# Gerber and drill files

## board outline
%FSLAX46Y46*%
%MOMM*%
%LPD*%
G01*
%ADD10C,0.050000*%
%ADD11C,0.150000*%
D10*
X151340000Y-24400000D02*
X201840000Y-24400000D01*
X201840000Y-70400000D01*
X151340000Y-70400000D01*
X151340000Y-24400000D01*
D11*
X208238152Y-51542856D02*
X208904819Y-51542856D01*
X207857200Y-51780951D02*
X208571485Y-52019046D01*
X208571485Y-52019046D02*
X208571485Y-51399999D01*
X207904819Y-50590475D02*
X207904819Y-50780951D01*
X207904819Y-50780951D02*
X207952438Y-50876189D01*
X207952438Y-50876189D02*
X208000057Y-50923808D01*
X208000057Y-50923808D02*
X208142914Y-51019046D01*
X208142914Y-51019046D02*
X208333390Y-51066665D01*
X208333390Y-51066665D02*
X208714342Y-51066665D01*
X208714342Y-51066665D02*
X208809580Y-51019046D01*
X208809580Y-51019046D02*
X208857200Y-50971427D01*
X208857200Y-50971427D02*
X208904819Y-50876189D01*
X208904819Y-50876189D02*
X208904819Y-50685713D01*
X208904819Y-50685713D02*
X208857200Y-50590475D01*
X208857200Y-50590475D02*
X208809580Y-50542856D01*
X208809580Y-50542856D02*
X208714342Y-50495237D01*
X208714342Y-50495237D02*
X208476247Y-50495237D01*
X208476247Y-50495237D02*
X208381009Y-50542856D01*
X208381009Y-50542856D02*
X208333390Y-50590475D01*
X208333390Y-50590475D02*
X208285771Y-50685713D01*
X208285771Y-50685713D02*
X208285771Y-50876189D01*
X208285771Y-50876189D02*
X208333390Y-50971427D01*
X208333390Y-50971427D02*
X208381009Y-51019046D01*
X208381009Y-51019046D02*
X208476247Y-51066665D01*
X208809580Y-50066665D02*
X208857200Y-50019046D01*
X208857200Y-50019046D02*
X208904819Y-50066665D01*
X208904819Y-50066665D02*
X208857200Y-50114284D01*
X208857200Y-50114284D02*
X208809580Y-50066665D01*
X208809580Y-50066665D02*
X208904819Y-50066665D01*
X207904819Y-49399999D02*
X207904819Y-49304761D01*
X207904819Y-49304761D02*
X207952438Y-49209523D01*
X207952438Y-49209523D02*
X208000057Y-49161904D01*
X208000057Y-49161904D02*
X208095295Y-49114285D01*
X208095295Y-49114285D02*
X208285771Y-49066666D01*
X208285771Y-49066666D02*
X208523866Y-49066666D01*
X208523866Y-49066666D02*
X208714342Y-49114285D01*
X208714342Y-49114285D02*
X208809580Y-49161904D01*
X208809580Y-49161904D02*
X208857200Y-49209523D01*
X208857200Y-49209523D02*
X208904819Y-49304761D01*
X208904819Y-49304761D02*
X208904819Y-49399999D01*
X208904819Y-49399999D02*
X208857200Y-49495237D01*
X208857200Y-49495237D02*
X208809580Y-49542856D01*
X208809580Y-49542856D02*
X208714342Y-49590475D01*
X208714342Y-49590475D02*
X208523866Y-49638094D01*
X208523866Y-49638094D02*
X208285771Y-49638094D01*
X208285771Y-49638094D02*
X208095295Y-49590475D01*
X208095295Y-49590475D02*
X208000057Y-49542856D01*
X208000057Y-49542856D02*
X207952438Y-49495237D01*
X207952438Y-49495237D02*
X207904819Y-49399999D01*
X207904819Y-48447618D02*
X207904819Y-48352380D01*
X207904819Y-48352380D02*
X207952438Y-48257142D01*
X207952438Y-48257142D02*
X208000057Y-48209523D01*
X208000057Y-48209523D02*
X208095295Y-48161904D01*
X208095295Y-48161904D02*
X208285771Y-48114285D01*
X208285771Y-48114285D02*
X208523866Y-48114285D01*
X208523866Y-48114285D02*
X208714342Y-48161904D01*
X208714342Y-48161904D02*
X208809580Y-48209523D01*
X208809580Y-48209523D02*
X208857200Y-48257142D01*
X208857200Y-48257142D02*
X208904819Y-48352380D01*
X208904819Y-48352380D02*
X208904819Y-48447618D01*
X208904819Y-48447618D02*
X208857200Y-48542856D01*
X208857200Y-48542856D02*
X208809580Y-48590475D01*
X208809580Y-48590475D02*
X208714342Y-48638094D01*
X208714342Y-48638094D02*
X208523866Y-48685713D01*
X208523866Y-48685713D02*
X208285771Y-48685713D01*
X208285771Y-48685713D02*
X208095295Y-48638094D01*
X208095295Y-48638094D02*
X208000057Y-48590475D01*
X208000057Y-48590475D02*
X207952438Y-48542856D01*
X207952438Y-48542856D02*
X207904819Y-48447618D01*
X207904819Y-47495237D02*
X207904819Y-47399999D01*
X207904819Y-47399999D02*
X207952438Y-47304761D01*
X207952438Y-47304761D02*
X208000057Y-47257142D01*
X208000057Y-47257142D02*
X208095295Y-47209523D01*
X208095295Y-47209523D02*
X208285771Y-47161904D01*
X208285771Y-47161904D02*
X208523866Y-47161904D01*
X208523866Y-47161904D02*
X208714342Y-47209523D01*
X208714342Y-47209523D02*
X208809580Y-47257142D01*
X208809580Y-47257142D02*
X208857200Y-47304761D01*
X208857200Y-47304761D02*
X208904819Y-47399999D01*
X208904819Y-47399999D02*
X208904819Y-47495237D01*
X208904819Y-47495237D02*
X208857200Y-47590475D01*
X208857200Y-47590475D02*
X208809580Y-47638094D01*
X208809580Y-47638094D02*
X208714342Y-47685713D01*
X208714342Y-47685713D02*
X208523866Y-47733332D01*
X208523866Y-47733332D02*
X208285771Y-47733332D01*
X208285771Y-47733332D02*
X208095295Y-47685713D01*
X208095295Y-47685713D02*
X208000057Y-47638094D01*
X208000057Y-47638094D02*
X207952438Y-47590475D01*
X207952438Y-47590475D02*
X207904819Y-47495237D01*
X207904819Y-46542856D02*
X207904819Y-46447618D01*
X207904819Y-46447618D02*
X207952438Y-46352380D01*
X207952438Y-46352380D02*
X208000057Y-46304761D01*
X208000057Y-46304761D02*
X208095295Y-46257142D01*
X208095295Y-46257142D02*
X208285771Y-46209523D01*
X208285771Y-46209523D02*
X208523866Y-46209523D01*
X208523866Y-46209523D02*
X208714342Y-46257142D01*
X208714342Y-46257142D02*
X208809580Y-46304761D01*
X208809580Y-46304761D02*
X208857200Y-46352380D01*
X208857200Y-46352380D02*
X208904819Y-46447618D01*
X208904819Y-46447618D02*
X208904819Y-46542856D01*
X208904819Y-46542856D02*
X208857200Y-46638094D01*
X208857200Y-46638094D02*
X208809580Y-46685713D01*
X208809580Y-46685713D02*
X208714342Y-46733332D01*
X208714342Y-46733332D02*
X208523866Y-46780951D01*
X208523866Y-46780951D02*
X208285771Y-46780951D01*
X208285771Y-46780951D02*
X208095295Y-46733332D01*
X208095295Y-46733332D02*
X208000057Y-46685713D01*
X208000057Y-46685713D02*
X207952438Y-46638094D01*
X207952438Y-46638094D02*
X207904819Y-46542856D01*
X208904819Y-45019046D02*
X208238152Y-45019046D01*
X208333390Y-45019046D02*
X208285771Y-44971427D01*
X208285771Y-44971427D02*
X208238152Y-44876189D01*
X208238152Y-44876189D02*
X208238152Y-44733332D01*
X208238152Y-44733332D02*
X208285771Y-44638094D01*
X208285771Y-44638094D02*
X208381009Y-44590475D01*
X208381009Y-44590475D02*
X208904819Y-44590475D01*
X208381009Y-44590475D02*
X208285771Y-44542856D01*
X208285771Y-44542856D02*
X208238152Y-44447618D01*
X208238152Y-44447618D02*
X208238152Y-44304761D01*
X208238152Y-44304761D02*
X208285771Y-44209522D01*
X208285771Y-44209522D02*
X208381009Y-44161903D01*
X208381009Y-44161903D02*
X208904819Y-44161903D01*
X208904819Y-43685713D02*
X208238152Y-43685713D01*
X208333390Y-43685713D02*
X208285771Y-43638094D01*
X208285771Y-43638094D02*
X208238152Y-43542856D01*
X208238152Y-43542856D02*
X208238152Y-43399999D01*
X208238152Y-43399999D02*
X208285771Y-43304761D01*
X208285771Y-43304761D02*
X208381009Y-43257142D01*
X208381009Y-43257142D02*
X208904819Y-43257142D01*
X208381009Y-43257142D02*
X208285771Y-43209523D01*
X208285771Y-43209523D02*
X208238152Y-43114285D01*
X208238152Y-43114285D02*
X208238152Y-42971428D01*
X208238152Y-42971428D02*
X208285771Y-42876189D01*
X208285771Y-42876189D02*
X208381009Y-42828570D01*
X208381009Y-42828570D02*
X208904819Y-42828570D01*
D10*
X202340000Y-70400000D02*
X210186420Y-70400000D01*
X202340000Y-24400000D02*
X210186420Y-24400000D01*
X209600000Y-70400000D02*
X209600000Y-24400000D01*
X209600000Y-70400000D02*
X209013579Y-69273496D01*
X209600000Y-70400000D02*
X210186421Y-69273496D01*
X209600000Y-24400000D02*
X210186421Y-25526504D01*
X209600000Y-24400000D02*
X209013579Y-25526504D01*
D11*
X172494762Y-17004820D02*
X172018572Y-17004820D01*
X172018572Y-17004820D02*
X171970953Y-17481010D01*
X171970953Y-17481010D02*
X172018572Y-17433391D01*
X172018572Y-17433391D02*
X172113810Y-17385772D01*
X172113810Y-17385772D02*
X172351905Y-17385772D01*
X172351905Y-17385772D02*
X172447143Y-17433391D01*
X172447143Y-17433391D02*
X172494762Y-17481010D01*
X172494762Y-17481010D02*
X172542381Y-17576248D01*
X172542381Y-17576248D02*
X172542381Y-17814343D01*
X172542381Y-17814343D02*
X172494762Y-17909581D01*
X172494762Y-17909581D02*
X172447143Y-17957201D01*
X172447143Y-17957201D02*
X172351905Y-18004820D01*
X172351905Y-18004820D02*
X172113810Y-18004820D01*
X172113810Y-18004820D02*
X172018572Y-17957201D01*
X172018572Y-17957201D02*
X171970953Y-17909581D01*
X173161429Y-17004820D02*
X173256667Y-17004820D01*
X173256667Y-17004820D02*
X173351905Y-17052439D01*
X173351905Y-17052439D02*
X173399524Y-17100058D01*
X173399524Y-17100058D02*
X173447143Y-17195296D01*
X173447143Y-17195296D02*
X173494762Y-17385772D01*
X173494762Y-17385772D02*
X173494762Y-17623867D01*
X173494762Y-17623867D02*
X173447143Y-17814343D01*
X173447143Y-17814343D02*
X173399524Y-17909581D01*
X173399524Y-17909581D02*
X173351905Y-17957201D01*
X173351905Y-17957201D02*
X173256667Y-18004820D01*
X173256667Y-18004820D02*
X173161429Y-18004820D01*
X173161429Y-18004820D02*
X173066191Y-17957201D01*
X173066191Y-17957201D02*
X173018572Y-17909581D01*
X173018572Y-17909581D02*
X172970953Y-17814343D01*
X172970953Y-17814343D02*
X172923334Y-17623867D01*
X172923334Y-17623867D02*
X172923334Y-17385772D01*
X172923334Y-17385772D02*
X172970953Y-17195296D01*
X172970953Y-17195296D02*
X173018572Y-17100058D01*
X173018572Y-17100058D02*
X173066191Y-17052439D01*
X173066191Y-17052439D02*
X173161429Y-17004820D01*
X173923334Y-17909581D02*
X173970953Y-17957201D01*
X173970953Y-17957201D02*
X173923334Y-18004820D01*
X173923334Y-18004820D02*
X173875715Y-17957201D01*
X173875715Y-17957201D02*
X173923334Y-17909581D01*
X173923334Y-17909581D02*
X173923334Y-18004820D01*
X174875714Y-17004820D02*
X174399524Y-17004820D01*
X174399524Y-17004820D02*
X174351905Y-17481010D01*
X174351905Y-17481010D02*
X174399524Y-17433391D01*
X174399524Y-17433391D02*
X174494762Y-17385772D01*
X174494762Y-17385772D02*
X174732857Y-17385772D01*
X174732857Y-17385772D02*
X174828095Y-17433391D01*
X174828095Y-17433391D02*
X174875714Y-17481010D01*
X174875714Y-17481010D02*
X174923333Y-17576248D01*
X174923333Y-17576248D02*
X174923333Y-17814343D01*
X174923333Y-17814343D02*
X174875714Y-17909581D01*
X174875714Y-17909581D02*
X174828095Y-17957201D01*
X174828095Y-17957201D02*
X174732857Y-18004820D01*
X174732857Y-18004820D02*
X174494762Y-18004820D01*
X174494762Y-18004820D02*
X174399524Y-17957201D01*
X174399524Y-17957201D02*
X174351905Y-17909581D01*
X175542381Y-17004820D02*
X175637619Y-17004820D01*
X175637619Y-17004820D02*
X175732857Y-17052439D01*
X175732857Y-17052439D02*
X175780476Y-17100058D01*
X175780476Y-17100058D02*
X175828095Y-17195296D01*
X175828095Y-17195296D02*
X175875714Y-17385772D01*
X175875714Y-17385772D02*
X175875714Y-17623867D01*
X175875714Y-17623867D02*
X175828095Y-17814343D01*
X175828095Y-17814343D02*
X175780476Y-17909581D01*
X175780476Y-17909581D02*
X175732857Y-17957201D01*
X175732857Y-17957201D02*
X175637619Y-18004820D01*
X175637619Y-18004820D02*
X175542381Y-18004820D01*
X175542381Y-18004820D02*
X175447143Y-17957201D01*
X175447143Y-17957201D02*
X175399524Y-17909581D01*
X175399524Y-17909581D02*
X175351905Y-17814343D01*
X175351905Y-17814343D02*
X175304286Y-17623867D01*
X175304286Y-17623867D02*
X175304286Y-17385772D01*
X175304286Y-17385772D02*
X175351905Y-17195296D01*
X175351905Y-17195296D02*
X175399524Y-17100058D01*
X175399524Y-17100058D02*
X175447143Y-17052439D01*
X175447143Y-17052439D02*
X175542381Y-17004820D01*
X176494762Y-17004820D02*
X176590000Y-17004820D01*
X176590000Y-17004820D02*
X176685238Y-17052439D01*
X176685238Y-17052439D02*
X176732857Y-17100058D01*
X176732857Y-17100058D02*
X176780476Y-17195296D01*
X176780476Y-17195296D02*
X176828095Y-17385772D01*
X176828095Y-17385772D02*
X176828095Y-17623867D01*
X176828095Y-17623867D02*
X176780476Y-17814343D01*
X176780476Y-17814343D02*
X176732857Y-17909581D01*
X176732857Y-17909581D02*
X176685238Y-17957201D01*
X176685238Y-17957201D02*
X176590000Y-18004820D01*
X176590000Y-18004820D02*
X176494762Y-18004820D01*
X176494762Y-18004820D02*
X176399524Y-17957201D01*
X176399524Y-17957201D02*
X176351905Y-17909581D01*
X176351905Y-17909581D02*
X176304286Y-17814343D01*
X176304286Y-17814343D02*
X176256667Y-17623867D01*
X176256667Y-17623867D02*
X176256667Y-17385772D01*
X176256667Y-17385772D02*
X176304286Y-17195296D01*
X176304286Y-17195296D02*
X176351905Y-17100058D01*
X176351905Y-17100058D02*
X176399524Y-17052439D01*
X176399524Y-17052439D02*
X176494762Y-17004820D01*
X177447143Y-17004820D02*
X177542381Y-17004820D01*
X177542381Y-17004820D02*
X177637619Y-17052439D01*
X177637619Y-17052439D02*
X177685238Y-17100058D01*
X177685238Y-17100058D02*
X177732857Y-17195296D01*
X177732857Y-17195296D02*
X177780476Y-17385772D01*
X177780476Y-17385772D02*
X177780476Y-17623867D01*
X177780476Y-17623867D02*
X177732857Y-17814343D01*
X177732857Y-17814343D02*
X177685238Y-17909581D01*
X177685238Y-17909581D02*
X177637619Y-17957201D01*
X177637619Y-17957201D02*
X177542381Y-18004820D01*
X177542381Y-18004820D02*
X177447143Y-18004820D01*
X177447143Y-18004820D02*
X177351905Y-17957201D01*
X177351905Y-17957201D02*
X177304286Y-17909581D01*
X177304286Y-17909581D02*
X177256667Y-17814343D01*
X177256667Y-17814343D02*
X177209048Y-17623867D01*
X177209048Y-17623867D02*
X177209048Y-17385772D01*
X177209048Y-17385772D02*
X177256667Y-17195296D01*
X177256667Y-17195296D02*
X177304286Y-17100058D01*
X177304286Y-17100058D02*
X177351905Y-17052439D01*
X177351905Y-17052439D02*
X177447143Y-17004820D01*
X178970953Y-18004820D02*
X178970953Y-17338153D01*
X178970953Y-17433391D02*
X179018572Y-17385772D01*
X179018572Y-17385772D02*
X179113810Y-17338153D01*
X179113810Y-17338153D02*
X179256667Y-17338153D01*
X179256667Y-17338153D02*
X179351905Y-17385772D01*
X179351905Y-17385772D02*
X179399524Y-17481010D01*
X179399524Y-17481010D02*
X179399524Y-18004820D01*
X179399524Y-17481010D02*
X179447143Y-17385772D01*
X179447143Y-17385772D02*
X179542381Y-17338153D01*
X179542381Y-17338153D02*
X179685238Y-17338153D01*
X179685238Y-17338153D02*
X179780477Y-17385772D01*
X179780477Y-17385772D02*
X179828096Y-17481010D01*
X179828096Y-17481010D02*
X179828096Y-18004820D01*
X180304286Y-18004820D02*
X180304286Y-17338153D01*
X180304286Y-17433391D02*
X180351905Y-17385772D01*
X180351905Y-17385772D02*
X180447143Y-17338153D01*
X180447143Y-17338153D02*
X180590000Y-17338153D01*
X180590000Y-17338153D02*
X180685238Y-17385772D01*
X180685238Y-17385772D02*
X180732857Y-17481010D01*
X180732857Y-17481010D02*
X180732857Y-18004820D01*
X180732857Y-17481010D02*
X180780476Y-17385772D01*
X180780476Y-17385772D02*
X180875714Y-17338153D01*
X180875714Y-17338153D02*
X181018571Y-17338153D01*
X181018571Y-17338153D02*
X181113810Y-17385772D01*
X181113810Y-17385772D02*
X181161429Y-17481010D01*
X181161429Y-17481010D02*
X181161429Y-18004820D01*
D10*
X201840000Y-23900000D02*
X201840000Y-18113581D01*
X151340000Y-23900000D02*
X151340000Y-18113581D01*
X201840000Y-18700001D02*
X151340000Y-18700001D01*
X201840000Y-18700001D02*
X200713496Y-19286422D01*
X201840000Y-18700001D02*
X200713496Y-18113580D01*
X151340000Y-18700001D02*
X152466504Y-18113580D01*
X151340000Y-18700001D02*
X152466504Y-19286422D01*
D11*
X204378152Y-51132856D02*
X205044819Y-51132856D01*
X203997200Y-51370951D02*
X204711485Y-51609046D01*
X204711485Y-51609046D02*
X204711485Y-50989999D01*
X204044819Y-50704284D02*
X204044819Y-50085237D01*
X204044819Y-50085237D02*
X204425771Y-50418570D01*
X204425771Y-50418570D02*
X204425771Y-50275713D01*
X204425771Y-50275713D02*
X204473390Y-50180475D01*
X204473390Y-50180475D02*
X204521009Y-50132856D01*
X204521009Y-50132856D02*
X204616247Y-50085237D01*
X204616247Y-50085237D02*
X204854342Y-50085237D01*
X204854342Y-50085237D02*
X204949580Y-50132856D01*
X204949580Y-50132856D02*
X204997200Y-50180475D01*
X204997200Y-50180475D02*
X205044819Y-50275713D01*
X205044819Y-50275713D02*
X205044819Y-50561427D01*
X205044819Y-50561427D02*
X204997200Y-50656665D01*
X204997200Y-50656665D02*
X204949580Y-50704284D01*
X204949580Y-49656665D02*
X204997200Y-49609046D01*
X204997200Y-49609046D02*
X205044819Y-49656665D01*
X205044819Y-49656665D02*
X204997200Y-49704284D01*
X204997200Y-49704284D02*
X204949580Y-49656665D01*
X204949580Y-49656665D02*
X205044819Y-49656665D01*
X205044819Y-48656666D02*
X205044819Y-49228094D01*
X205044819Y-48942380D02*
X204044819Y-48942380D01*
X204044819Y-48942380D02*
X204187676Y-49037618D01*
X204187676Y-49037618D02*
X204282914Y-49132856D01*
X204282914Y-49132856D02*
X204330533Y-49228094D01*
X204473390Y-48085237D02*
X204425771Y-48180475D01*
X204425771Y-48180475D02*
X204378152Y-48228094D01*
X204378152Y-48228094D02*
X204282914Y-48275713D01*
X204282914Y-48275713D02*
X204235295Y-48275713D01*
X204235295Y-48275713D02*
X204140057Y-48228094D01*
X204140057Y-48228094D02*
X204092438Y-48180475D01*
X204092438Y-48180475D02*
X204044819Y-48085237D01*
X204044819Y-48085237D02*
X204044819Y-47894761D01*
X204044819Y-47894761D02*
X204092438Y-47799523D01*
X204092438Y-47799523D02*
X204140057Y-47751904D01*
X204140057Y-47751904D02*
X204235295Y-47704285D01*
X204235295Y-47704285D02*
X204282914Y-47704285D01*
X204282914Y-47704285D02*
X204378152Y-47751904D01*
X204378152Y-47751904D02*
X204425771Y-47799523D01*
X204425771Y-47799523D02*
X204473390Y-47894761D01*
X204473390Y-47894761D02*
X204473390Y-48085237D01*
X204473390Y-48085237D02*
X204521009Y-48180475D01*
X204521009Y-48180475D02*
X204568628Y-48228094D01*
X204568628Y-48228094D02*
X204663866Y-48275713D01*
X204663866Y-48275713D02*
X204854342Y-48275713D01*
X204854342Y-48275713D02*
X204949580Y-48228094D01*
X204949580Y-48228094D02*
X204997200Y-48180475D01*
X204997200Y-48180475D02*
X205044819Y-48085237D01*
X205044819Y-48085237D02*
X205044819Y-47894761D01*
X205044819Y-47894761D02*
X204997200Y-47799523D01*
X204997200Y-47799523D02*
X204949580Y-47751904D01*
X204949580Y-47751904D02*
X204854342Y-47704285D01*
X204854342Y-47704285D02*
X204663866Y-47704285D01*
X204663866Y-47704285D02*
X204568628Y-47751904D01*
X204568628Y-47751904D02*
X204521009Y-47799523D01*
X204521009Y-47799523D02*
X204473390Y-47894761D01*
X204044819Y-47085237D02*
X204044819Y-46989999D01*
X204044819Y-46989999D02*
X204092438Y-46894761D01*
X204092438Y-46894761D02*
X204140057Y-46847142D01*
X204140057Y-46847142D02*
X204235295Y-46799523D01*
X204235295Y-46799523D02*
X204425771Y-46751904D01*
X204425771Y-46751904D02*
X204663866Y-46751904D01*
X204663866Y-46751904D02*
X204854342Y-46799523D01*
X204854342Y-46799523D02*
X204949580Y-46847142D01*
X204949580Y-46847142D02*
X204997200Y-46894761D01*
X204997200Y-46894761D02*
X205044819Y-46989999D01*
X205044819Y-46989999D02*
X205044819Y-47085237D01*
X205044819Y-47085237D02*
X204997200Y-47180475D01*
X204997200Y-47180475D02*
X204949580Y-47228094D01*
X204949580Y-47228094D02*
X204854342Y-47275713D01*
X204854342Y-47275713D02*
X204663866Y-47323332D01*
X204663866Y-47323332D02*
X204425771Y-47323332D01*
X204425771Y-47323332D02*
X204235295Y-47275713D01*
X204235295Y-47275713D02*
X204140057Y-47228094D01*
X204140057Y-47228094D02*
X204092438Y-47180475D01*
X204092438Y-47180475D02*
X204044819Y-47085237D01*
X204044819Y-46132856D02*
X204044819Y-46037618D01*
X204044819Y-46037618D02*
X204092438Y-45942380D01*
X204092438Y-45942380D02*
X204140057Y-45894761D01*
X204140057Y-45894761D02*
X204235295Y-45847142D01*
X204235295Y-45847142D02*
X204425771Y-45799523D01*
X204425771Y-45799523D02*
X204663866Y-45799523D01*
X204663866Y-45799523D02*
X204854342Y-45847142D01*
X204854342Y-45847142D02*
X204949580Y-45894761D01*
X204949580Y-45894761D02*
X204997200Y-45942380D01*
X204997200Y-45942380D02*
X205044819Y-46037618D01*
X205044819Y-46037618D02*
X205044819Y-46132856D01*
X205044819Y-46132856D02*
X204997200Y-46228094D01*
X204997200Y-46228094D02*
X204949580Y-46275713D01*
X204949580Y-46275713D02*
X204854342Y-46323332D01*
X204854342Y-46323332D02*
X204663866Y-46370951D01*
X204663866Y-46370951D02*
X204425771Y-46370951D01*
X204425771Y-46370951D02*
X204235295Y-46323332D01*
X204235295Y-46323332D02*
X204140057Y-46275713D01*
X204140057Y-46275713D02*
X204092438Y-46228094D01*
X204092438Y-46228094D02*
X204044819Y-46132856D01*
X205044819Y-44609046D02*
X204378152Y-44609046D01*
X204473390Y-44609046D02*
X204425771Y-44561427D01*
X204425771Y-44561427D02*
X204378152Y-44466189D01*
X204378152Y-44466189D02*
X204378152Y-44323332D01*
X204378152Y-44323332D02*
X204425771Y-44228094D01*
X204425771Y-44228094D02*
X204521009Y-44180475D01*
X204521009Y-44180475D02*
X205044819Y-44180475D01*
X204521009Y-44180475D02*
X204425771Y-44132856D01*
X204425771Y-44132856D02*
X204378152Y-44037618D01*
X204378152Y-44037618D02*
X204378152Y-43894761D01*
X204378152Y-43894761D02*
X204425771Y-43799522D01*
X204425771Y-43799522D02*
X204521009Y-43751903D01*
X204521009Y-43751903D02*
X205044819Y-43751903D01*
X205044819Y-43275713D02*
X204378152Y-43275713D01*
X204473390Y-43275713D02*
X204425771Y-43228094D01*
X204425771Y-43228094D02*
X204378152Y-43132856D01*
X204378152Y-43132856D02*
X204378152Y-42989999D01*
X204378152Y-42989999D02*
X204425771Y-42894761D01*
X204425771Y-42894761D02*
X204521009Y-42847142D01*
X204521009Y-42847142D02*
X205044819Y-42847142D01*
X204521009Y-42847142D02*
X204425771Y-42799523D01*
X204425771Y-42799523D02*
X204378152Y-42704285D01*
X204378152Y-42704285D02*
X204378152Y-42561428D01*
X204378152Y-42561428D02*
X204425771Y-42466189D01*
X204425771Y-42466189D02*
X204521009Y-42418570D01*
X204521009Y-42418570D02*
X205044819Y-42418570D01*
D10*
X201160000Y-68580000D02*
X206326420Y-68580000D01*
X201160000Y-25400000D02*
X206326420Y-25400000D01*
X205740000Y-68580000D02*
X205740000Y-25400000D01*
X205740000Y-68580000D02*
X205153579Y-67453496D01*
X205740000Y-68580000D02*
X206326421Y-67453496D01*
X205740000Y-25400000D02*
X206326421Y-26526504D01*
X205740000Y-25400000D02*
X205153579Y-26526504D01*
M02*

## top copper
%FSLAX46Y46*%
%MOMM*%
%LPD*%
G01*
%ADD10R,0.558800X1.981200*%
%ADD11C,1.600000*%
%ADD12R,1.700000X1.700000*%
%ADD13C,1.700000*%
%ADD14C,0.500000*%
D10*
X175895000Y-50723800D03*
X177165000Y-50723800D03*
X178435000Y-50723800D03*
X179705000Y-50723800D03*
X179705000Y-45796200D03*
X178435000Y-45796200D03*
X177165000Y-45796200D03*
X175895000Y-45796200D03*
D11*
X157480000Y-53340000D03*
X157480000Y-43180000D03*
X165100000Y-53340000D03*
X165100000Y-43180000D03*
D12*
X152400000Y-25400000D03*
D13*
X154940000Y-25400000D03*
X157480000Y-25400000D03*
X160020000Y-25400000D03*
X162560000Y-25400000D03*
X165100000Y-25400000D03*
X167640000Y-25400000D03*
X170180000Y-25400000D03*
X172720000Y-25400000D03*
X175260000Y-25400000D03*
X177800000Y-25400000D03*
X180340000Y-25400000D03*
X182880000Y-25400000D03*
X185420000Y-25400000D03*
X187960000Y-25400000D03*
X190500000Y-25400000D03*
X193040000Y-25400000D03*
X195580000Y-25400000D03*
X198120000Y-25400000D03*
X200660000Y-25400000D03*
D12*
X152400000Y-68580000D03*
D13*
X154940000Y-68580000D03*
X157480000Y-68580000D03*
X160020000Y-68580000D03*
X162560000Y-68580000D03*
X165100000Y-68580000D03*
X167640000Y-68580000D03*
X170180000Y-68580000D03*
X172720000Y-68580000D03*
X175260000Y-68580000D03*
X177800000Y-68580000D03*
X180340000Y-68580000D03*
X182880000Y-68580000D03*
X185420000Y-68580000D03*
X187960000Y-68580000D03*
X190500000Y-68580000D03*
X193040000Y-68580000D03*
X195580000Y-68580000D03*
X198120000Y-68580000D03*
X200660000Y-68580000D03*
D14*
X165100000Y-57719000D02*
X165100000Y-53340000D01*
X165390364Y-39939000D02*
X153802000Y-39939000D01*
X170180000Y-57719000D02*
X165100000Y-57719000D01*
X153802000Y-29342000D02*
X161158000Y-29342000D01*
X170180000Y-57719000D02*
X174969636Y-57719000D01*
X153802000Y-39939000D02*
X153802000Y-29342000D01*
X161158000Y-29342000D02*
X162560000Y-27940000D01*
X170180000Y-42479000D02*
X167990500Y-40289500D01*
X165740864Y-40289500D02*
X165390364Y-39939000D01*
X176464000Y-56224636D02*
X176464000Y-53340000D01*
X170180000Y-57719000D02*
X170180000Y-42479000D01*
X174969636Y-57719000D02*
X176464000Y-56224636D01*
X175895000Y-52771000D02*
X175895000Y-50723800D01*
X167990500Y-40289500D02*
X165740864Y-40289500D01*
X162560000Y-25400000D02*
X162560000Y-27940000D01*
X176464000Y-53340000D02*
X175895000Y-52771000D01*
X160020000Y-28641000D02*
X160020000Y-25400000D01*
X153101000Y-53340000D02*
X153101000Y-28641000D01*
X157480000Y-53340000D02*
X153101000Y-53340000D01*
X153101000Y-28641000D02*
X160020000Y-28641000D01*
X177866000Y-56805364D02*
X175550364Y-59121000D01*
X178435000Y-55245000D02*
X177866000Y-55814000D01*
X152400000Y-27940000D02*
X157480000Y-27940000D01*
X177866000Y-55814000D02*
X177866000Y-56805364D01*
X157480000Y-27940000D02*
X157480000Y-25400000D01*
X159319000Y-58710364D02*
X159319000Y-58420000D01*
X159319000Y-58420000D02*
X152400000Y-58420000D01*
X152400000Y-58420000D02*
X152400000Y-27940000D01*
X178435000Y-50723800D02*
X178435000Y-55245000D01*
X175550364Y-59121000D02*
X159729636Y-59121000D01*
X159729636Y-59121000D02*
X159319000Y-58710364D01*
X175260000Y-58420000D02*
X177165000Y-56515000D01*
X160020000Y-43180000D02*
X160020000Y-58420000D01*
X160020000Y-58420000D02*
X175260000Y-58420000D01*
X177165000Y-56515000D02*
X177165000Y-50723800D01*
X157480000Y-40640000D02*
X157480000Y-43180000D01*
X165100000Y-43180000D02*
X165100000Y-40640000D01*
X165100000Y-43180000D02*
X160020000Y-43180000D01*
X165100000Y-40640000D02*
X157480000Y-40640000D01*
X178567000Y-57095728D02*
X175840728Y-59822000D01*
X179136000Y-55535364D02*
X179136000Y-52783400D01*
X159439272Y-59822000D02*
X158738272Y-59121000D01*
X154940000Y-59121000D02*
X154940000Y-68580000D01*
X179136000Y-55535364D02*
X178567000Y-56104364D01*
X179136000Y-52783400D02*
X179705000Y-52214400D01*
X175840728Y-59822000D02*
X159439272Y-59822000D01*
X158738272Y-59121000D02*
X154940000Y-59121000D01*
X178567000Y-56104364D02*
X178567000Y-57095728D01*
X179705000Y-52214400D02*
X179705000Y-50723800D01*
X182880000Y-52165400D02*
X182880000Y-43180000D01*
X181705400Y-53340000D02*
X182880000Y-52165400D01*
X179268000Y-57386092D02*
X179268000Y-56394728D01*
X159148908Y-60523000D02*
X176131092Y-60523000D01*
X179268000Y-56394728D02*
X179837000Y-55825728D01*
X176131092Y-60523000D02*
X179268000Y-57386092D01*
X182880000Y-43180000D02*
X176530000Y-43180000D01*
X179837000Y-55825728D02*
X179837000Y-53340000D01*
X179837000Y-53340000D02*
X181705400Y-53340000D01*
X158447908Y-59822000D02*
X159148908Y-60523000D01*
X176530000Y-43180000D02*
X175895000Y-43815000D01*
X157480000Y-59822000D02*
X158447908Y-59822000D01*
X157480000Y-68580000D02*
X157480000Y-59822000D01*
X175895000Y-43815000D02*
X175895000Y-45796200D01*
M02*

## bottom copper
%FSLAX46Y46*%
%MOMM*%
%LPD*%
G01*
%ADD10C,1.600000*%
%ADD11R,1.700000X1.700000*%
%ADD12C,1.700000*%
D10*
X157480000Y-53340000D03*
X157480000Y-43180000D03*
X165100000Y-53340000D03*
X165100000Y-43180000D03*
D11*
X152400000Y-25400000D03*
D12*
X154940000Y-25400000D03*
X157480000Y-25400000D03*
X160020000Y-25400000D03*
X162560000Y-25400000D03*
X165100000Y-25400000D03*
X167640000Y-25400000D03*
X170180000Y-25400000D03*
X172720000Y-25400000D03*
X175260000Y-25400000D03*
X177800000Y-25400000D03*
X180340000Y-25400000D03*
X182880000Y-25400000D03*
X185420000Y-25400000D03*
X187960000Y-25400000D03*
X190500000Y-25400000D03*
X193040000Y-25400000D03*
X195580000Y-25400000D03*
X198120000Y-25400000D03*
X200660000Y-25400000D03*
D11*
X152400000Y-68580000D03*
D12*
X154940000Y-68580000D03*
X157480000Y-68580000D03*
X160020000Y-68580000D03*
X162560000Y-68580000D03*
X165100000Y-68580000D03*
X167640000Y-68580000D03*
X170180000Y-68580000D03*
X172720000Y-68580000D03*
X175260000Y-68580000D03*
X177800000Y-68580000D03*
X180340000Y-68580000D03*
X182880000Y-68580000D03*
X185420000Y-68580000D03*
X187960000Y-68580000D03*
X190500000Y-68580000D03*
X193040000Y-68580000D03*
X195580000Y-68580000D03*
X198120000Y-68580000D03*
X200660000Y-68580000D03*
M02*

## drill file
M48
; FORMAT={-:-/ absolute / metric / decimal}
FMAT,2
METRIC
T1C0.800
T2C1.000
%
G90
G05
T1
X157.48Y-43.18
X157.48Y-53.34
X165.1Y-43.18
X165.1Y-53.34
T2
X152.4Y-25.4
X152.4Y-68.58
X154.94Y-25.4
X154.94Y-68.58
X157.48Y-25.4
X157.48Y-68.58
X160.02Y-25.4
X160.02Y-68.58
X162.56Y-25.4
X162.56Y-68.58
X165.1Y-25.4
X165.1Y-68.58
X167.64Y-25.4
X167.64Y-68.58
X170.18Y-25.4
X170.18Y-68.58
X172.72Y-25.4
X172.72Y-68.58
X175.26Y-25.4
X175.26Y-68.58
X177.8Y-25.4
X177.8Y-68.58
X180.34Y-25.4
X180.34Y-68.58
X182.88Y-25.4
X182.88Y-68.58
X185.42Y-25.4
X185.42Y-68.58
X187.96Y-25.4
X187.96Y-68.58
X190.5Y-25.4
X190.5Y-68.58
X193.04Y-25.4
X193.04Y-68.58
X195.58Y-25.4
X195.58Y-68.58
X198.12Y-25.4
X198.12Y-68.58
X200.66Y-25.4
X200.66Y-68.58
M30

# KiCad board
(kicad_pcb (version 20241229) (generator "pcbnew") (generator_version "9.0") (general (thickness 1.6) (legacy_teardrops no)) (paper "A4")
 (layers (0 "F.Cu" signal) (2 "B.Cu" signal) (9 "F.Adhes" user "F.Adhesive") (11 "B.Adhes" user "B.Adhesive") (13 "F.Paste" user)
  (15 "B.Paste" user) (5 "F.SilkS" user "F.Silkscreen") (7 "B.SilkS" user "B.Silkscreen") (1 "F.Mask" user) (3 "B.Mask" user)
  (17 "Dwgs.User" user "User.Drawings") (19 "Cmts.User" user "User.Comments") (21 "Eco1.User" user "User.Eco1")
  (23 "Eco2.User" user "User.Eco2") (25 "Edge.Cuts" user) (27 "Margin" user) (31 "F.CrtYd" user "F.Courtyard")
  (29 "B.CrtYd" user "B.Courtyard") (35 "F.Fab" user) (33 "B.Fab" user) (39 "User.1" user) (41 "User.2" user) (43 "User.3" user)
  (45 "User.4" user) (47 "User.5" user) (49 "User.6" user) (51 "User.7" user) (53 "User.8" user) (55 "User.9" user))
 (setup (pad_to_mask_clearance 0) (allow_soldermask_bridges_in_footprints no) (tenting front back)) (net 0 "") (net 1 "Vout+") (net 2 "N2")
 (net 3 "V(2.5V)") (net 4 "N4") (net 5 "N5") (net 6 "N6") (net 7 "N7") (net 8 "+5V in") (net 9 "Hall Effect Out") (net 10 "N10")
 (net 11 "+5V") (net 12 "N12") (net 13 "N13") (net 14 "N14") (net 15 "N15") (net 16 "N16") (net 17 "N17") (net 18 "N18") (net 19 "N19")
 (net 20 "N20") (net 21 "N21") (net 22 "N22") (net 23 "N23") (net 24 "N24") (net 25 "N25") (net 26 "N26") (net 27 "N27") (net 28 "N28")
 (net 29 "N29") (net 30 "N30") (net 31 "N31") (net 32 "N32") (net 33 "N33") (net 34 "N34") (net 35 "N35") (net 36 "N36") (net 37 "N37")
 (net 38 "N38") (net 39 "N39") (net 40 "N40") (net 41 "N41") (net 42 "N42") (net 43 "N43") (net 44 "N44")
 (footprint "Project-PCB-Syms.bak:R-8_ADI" (layer "F.Cu") (at 177.8 48.26 90)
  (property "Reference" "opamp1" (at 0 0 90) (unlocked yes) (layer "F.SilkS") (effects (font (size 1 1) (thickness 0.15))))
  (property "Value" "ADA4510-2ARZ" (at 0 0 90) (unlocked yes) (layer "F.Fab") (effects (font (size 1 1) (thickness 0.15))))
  (pad "1" smd rect (at -2.4638 -1.905 90) (size 1.9812 0.5588) (layers "F.Cu" "F.Mask" "F.Paste") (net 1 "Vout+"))
  (pad "2" smd rect (at -2.4638 -0.635 90) (size 1.9812 0.5588) (layers "F.Cu" "F.Mask" "F.Paste") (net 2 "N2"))
  (pad "3" smd rect (at -2.4638 0.635 90) (size 1.9812 0.5588) (layers "F.Cu" "F.Mask" "F.Paste") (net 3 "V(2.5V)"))
  (pad "4" smd rect (at -2.4638 1.905 90) (size 1.9812 0.5588) (layers "F.Cu" "F.Mask" "F.Paste") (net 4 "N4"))
  (pad "5" smd rect (at 2.4638 1.905 90) (size 1.9812 0.5588) (layers "F.Cu" "F.Mask" "F.Paste") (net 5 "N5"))
  (pad "6" smd rect (at 2.4638 0.635 90) (size 1.9812 0.5588) (layers "F.Cu" "F.Mask" "F.Paste") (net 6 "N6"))
  (pad "7" smd rect (at 2.4638 -0.635 90) (size 1.9812 0.5588) (layers "F.Cu" "F.Mask" "F.Paste") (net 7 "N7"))
  (pad "8" smd rect (at 2.4638 -1.905 90) (size 1.9812 0.5588) (layers "F.Cu" "F.Mask" "F.Paste") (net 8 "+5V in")))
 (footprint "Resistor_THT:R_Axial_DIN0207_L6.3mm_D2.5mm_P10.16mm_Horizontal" (layer "F.Cu") (at 157.48 53.34 90)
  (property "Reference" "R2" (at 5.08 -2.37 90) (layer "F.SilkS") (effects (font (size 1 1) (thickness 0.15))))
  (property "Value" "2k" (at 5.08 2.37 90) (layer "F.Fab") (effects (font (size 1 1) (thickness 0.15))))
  (pad "1" thru_hole circle (at 0 0 90) (size 1.6 1.6) (drill 0.8) (layers "*.Cu" "*.Mask") (remove_unused_layers no)
   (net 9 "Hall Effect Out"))
  (pad "2" thru_hole circle (at 10.16 0 90) (size 1.6 1.6) (drill 0.8) (layers "*.Cu" "*.Mask") (remove_unused_layers no) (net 2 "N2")))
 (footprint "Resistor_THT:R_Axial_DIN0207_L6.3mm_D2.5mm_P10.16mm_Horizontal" (layer "F.Cu") (at 165.1 53.34 90)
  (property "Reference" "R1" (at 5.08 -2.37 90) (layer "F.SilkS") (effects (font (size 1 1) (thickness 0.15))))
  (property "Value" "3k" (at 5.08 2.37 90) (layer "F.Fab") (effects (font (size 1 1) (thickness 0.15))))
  (pad "1" thru_hole circle (at 0 0 90) (size 1.6 1.6) (drill 0.8) (layers "*.Cu" "*.Mask") (remove_unused_layers no) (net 1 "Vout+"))
  (pad "2" thru_hole circle (at 10.16 0 90) (size 1.6 1.6) (drill 0.8) (layers "*.Cu" "*.Mask") (remove_unused_layers no) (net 2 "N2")))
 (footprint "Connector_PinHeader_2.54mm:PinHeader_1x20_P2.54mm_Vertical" (layer "F.Cu") (at 152.4 25.4 90)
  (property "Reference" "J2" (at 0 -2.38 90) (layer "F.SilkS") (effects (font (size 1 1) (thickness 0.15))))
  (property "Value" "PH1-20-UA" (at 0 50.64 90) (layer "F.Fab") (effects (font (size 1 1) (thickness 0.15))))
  (pad "1" thru_hole rect (at 0 0 90) (size 1.7 1.7) (drill 1) (layers "*.Cu" "*.Mask") (remove_unused_layers no) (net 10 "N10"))
  (pad "2" thru_hole circle (at 0 2.54 90) (size 1.7 1.7) (drill 1) (layers "*.Cu" "*.Mask") (remove_unused_layers no) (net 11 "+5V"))
  (pad "3" thru_hole circle (at 0 5.08 90) (size 1.7 1.7) (drill 1) (layers "*.Cu" "*.Mask") (remove_unused_layers no) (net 3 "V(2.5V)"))
  (pad "4" thru_hole circle (at 0 7.62 90) (size 1.7 1.7) (drill 1) (layers "*.Cu" "*.Mask") (remove_unused_layers no)
   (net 9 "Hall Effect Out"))
  (pad "5" thru_hole circle (at 0 10.16 90) (size 1.7 1.7) (drill 1) (layers "*.Cu" "*.Mask") (remove_unused_layers no) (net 1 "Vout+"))
  (pad "6" thru_hole circle (at 0 12.7 90) (size 1.7 1.7) (drill 1) (layers "*.Cu" "*.Mask") (remove_unused_layers no) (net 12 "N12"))
  (pad "7" thru_hole circle (at 0 15.24 90) (size 1.7 1.7) (drill 1) (layers "*.Cu" "*.Mask") (remove_unused_layers no) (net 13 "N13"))
  (pad "8" thru_hole circle (at 0 17.78 90) (size 1.7 1.7) (drill 1) (layers "*.Cu" "*.Mask") (remove_unused_layers no) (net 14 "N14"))
  (pad "9" thru_hole circle (at 0 20.32 90) (size 1.7 1.7) (drill 1) (layers "*.Cu" "*.Mask") (remove_unused_layers no) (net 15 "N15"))
  (pad "10" thru_hole circle (at 0 22.86 90) (size 1.7 1.7) (drill 1) (layers "*.Cu" "*.Mask") (remove_unused_layers no) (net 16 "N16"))
  (pad "11" thru_hole circle (at 0 25.4 90) (size 1.7 1.7) (drill 1) (layers "*.Cu" "*.Mask") (remove_unused_layers no) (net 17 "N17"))
  (pad "12" thru_hole circle (at 0 27.94 90) (size 1.7 1.7) (drill 1) (layers "*.Cu" "*.Mask") (remove_unused_layers no) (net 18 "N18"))
  (pad "13" thru_hole circle (at 0 30.48 90) (size 1.7 1.7) (drill 1) (layers "*.Cu" "*.Mask") (remove_unused_layers no) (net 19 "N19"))
  (pad "14" thru_hole circle (at 0 33.02 90) (size 1.7 1.7) (drill 1) (layers "*.Cu" "*.Mask") (remove_unused_layers no) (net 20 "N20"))
  (pad "15" thru_hole circle (at 0 35.56 90) (size 1.7 1.7) (drill 1) (layers "*.Cu" "*.Mask") (remove_unused_layers no) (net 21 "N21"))
  (pad "16" thru_hole circle (at 0 38.1 90) (size 1.7 1.7) (drill 1) (layers "*.Cu" "*.Mask") (remove_unused_layers no) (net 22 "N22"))
  (pad "17" thru_hole circle (at 0 40.64 90) (size 1.7 1.7) (drill 1) (layers "*.Cu" "*.Mask") (remove_unused_layers no) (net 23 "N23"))
  (pad "18" thru_hole circle (at 0 43.18 90) (size 1.7 1.7) (drill 1) (layers "*.Cu" "*.Mask") (remove_unused_layers no) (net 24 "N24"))
  (pad "19" thru_hole circle (at 0 45.72 90) (size 1.7 1.7) (drill 1) (layers "*.Cu" "*.Mask") (remove_unused_layers no) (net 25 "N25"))
  (pad "20" thru_hole circle (at 0 48.26 90) (size 1.7 1.7) (drill 1) (layers "*.Cu" "*.Mask") (remove_unused_layers no) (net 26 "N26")))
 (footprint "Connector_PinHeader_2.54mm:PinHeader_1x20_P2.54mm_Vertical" (layer "F.Cu") (at 152.4 68.58 90)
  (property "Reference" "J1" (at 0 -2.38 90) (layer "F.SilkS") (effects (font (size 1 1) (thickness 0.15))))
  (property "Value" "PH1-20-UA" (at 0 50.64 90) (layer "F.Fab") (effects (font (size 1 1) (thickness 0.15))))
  (pad "1" thru_hole rect (at 0 0 90) (size 1.7 1.7) (drill 1) (layers "*.Cu" "*.Mask") (remove_unused_layers no) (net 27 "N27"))
  (pad "2" thru_hole circle (at 0 2.54 90) (size 1.7 1.7) (drill 1) (layers "*.Cu" "*.Mask") (remove_unused_layers no) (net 4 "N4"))
  (pad "3" thru_hole circle (at 0 5.08 90) (size 1.7 1.7) (drill 1) (layers "*.Cu" "*.Mask") (remove_unused_layers no) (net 8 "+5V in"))
  (pad "4" thru_hole circle (at 0 7.62 90) (size 1.7 1.7) (drill 1) (layers "*.Cu" "*.Mask") (remove_unused_layers no) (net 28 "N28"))
  (pad "5" thru_hole circle (at 0 10.16 90) (size 1.7 1.7) (drill 1) (layers "*.Cu" "*.Mask") (remove_unused_layers no) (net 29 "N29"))
  (pad "6" thru_hole circle (at 0 12.7 90) (size 1.7 1.7) (drill 1) (layers "*.Cu" "*.Mask") (remove_unused_layers no) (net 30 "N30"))
  (pad "7" thru_hole circle (at 0 15.24 90) (size 1.7 1.7) (drill 1) (layers "*.Cu" "*.Mask") (remove_unused_layers no) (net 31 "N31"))
  (pad "8" thru_hole circle (at 0 17.78 90) (size 1.7 1.7) (drill 1) (layers "*.Cu" "*.Mask") (remove_unused_layers no) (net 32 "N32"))
  (pad "9" thru_hole circle (at 0 20.32 90) (size 1.7 1.7) (drill 1) (layers "*.Cu" "*.Mask") (remove_unused_layers no) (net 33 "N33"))
  (pad "10" thru_hole circle (at 0 22.86 90) (size 1.7 1.7) (drill 1) (layers "*.Cu" "*.Mask") (remove_unused_layers no) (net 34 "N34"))
  (pad "11" thru_hole circle (at 0 25.4 90) (size 1.7 1.7) (drill 1) (layers "*.Cu" "*.Mask") (remove_unused_layers no) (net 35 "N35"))
  (pad "12" thru_hole circle (at 0 27.94 90) (size 1.7 1.7) (drill 1) (layers "*.Cu" "*.Mask") (remove_unused_layers no) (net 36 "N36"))
  (pad "13" thru_hole circle (at 0 30.48 90) (size 1.7 1.7) (drill 1) (layers "*.Cu" "*.Mask") (remove_unused_layers no) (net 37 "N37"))
  (pad "14" thru_hole circle (at 0 33.02 90) (size 1.7 1.7) (drill 1) (layers "*.Cu" "*.Mask") (remove_unused_layers no) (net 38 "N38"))
  (pad "15" thru_hole circle (at 0 35.56 90) (size 1.7 1.7) (drill 1) (layers "*.Cu" "*.Mask") (remove_unused_layers no) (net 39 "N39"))
  (pad "16" thru_hole circle (at 0 38.1 90) (size 1.7 1.7) (drill 1) (layers "*.Cu" "*.Mask") (remove_unused_layers no) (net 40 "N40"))
  (pad "17" thru_hole circle (at 0 40.64 90) (size 1.7 1.7) (drill 1) (layers "*.Cu" "*.Mask") (remove_unused_layers no) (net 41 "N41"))
  (pad "18" thru_hole circle (at 0 43.18 90) (size 1.7 1.7) (drill 1) (layers "*.Cu" "*.Mask") (remove_unused_layers no) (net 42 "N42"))
  (pad "19" thru_hole circle (at 0 45.72 90) (size 1.7 1.7) (drill 1) (layers "*.Cu" "*.Mask") (remove_unused_layers no) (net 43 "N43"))
  (pad "20" thru_hole circle (at 0 48.26 90) (size 1.7 1.7) (drill 1) (layers "*.Cu" "*.Mask") (remove_unused_layers no) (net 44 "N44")))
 (gr_rect (start 151.34 24.4) (end 201.84 70.4) (stroke (width 0.05) (type default)) (fill no) (layer "Edge.Cuts"))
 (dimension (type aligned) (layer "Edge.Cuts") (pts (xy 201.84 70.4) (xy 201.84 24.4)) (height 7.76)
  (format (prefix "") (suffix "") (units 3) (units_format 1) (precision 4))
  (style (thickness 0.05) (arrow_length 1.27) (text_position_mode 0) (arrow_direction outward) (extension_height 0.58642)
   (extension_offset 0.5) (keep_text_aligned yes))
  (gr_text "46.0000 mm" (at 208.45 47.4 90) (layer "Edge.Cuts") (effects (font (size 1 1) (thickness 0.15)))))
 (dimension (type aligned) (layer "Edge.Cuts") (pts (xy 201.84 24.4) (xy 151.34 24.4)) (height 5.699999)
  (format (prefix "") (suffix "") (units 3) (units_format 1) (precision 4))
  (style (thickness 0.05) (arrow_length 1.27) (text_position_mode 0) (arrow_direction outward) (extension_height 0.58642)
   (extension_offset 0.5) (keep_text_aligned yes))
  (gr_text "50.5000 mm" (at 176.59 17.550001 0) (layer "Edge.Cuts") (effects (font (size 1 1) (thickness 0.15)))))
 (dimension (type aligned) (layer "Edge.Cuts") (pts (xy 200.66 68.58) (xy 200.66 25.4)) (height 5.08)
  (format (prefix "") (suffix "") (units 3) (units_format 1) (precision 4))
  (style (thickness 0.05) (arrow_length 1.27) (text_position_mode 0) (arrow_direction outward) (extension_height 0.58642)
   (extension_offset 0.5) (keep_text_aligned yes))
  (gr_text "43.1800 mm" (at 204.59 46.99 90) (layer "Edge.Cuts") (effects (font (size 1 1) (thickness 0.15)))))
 (segment (start 165.1 57.719) (end 165.1 53.34) (width 0.5) (layer "F.Cu") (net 1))
 (segment (start 165.390364 39.939) (end 153.802 39.939) (width 0.5) (layer "F.Cu") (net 1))
 (segment (start 170.18 57.719) (end 165.1 57.719) (width 0.5) (layer "F.Cu") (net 1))
 (segment (start 153.802 29.342) (end 161.158 29.342) (width 0.5) (layer "F.Cu") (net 1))
 (segment (start 170.18 57.719) (end 174.969636 57.719) (width 0.5) (layer "F.Cu") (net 1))
 (segment (start 153.802 39.939) (end 153.802 29.342) (width 0.5) (layer "F.Cu") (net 1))
 (segment (start 161.158 29.342) (end 162.56 27.94) (width 0.5) (layer "F.Cu") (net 1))
 (segment (start 170.18 42.479) (end 167.9905 40.2895) (width 0.5) (layer "F.Cu") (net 1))
 (segment (start 165.740864 40.2895) (end 165.390364 39.939) (width 0.5) (layer "F.Cu") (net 1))
 (segment (start 176.464 56.224636) (end 176.464 53.34) (width 0.5) (layer "F.Cu") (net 1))
 (segment (start 170.18 57.719) (end 170.18 42.479) (width 0.5) (layer "F.Cu") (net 1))
 (segment (start 174.969636 57.719) (end 176.464 56.224636) (width 0.5) (layer "F.Cu") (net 1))
 (segment (start 175.895 52.771) (end 175.895 50.7238) (width 0.5) (layer "F.Cu") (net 1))
 (segment (start 167.9905 40.2895) (end 165.740864 40.2895) (width 0.5) (layer "F.Cu") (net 1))
 (segment (start 162.56 25.4) (end 162.56 27.94) (width 0.5) (layer "F.Cu") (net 1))
 (segment (start 176.464 53.34) (end 175.895 52.771) (width 0.5) (layer "F.Cu") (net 1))
 (segment (start 160.02 28.641) (end 160.02 25.4) (width 0.5) (layer "F.Cu") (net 9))
 (segment (start 153.101 53.34) (end 153.101 28.641) (width 0.5) (layer "F.Cu") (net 9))
 (segment (start 157.48 53.34) (end 153.101 53.34) (width 0.5) (layer "F.Cu") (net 9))
 (segment (start 153.101 28.641) (end 160.02 28.641) (width 0.5) (layer "F.Cu") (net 9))
 (segment (start 177.866 56.805364) (end 175.550364 59.121) (width 0.5) (layer "F.Cu") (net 3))
 (segment (start 178.435 55.245) (end 177.866 55.814) (width 0.5) (layer "F.Cu") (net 3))
 (segment (start 152.4 27.94) (end 157.48 27.94) (width 0.5) (layer "F.Cu") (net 3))
 (segment (start 177.866 55.814) (end 177.866 56.805364) (width 0.5) (layer "F.Cu") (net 3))
 (segment (start 157.48 27.94) (end 157.48 25.4) (width 0.5) (layer "F.Cu") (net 3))
 (segment (start 159.319 58.710364) (end 159.319 58.42) (width 0.5) (layer "F.Cu") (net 3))
 (segment (start 159.319 58.42) (end 152.4 58.42) (width 0.5) (layer "F.Cu") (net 3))
 (segment (start 152.4 58.42) (end 152.4 27.94) (width 0.5) (layer "F.Cu") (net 3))
 (segment (start 178.435 50.7238) (end 178.435 55.245) (width 0.5) (layer "F.Cu") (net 3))
 (segment (start 175.550364 59.121) (end 159.729636 59.121) (width 0.5) (layer "F.Cu") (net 3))
 (segment (start 159.729636 59.121) (end 159.319 58.710364) (width 0.5) (layer "F.Cu") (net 3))
 (segment (start 175.26 58.42) (end 177.165 56.515) (width 0.5) (layer "F.Cu") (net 2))
 (segment (start 160.02 43.18) (end 160.02 58.42) (width 0.5) (layer "F.Cu") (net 2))
 (segment (start 160.02 58.42) (end 175.26 58.42) (width 0.5) (layer "F.Cu") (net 2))
 (segment (start 177.165 56.515) (end 177.165 50.7238) (width 0.5) (layer "F.Cu") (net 2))
 (segment (start 157.48 40.64) (end 157.48 43.18) (width 0.5) (layer "F.Cu") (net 2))
 (segment (start 165.1 43.18) (end 165.1 40.64) (width 0.5) (layer "F.Cu") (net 2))
 (segment (start 165.1 43.18) (end 160.02 43.18) (width 0.5) (layer "F.Cu") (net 2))
 (segment (start 165.1 40.64) (end 157.48 40.64) (width 0.5) (layer "F.Cu") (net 2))
 (segment (start 178.567 57.095728) (end 175.840728 59.822) (width 0.5) (layer "F.Cu") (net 4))
 (segment (start 179.136 55.535364) (end 179.136 52.7834) (width 0.5) (layer "F.Cu") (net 4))
 (segment (start 159.439272 59.822) (end 158.738272 59.121) (width 0.5) (layer "F.Cu") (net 4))
 (segment (start 154.94 59.121) (end 154.94 68.58) (width 0.5) (layer "F.Cu") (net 4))
 (segment (start 179.136 55.535364) (end 178.567 56.104364) (width 0.5) (layer "F.Cu") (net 4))
 (segment (start 179.136 52.7834) (end 179.705 52.2144) (width 0.5) (layer "F.Cu") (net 4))
 (segment (start 175.840728 59.822) (end 159.439272 59.822) (width 0.5) (layer "F.Cu") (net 4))
 (segment (start 158.738272 59.121) (end 154.94 59.121) (width 0.5) (layer "F.Cu") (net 4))
 (segment (start 178.567 56.104364) (end 178.567 57.095728) (width 0.5) (layer "F.Cu") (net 4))
 (segment (start 179.705 52.2144) (end 179.705 50.7238) (width 0.5) (layer "F.Cu") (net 4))
 (segment (start 182.88 52.1654) (end 182.88 43.18) (width 0.5) (layer "F.Cu") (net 8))
 (segment (start 181.7054 53.34) (end 182.88 52.1654) (width 0.5) (layer "F.Cu") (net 8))
 (segment (start 179.268 57.386092) (end 179.268 56.394728) (width 0.5) (layer "F.Cu") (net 8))
 (segment (start 159.148908 60.523) (end 176.131092 60.523) (width 0.5) (layer "F.Cu") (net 8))
 (segment (start 179.268 56.394728) (end 179.837 55.825728) (width 0.5) (layer "F.Cu") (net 8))
 (segment (start 176.131092 60.523) (end 179.268 57.386092) (width 0.5) (layer "F.Cu") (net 8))
 (segment (start 182.88 43.18) (end 176.53 43.18) (width 0.5) (layer "F.Cu") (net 8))
 (segment (start 179.837 55.825728) (end 179.837 53.34) (width 0.5) (layer "F.Cu") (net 8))
 (segment (start 179.837 53.34) (end 181.7054 53.34) (width 0.5) (layer "F.Cu") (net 8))
 (segment (start 158.447908 59.822) (end 159.148908 60.523) (width 0.5) (layer "F.Cu") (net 8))
 (segment (start 176.53 43.18) (end 175.895 43.815) (width 0.5) (layer "F.Cu") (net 8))
 (segment (start 157.48 59.822) (end 158.447908 59.822) (width 0.5) (layer "F.Cu") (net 8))
 (segment (start 157.48 68.58) (end 157.48 59.822) (width 0.5) (layer "F.Cu") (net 8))
 (segment (start 175.895 43.815) (end 175.895 45.7962) (width 0.5) (layer "F.Cu") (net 8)))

